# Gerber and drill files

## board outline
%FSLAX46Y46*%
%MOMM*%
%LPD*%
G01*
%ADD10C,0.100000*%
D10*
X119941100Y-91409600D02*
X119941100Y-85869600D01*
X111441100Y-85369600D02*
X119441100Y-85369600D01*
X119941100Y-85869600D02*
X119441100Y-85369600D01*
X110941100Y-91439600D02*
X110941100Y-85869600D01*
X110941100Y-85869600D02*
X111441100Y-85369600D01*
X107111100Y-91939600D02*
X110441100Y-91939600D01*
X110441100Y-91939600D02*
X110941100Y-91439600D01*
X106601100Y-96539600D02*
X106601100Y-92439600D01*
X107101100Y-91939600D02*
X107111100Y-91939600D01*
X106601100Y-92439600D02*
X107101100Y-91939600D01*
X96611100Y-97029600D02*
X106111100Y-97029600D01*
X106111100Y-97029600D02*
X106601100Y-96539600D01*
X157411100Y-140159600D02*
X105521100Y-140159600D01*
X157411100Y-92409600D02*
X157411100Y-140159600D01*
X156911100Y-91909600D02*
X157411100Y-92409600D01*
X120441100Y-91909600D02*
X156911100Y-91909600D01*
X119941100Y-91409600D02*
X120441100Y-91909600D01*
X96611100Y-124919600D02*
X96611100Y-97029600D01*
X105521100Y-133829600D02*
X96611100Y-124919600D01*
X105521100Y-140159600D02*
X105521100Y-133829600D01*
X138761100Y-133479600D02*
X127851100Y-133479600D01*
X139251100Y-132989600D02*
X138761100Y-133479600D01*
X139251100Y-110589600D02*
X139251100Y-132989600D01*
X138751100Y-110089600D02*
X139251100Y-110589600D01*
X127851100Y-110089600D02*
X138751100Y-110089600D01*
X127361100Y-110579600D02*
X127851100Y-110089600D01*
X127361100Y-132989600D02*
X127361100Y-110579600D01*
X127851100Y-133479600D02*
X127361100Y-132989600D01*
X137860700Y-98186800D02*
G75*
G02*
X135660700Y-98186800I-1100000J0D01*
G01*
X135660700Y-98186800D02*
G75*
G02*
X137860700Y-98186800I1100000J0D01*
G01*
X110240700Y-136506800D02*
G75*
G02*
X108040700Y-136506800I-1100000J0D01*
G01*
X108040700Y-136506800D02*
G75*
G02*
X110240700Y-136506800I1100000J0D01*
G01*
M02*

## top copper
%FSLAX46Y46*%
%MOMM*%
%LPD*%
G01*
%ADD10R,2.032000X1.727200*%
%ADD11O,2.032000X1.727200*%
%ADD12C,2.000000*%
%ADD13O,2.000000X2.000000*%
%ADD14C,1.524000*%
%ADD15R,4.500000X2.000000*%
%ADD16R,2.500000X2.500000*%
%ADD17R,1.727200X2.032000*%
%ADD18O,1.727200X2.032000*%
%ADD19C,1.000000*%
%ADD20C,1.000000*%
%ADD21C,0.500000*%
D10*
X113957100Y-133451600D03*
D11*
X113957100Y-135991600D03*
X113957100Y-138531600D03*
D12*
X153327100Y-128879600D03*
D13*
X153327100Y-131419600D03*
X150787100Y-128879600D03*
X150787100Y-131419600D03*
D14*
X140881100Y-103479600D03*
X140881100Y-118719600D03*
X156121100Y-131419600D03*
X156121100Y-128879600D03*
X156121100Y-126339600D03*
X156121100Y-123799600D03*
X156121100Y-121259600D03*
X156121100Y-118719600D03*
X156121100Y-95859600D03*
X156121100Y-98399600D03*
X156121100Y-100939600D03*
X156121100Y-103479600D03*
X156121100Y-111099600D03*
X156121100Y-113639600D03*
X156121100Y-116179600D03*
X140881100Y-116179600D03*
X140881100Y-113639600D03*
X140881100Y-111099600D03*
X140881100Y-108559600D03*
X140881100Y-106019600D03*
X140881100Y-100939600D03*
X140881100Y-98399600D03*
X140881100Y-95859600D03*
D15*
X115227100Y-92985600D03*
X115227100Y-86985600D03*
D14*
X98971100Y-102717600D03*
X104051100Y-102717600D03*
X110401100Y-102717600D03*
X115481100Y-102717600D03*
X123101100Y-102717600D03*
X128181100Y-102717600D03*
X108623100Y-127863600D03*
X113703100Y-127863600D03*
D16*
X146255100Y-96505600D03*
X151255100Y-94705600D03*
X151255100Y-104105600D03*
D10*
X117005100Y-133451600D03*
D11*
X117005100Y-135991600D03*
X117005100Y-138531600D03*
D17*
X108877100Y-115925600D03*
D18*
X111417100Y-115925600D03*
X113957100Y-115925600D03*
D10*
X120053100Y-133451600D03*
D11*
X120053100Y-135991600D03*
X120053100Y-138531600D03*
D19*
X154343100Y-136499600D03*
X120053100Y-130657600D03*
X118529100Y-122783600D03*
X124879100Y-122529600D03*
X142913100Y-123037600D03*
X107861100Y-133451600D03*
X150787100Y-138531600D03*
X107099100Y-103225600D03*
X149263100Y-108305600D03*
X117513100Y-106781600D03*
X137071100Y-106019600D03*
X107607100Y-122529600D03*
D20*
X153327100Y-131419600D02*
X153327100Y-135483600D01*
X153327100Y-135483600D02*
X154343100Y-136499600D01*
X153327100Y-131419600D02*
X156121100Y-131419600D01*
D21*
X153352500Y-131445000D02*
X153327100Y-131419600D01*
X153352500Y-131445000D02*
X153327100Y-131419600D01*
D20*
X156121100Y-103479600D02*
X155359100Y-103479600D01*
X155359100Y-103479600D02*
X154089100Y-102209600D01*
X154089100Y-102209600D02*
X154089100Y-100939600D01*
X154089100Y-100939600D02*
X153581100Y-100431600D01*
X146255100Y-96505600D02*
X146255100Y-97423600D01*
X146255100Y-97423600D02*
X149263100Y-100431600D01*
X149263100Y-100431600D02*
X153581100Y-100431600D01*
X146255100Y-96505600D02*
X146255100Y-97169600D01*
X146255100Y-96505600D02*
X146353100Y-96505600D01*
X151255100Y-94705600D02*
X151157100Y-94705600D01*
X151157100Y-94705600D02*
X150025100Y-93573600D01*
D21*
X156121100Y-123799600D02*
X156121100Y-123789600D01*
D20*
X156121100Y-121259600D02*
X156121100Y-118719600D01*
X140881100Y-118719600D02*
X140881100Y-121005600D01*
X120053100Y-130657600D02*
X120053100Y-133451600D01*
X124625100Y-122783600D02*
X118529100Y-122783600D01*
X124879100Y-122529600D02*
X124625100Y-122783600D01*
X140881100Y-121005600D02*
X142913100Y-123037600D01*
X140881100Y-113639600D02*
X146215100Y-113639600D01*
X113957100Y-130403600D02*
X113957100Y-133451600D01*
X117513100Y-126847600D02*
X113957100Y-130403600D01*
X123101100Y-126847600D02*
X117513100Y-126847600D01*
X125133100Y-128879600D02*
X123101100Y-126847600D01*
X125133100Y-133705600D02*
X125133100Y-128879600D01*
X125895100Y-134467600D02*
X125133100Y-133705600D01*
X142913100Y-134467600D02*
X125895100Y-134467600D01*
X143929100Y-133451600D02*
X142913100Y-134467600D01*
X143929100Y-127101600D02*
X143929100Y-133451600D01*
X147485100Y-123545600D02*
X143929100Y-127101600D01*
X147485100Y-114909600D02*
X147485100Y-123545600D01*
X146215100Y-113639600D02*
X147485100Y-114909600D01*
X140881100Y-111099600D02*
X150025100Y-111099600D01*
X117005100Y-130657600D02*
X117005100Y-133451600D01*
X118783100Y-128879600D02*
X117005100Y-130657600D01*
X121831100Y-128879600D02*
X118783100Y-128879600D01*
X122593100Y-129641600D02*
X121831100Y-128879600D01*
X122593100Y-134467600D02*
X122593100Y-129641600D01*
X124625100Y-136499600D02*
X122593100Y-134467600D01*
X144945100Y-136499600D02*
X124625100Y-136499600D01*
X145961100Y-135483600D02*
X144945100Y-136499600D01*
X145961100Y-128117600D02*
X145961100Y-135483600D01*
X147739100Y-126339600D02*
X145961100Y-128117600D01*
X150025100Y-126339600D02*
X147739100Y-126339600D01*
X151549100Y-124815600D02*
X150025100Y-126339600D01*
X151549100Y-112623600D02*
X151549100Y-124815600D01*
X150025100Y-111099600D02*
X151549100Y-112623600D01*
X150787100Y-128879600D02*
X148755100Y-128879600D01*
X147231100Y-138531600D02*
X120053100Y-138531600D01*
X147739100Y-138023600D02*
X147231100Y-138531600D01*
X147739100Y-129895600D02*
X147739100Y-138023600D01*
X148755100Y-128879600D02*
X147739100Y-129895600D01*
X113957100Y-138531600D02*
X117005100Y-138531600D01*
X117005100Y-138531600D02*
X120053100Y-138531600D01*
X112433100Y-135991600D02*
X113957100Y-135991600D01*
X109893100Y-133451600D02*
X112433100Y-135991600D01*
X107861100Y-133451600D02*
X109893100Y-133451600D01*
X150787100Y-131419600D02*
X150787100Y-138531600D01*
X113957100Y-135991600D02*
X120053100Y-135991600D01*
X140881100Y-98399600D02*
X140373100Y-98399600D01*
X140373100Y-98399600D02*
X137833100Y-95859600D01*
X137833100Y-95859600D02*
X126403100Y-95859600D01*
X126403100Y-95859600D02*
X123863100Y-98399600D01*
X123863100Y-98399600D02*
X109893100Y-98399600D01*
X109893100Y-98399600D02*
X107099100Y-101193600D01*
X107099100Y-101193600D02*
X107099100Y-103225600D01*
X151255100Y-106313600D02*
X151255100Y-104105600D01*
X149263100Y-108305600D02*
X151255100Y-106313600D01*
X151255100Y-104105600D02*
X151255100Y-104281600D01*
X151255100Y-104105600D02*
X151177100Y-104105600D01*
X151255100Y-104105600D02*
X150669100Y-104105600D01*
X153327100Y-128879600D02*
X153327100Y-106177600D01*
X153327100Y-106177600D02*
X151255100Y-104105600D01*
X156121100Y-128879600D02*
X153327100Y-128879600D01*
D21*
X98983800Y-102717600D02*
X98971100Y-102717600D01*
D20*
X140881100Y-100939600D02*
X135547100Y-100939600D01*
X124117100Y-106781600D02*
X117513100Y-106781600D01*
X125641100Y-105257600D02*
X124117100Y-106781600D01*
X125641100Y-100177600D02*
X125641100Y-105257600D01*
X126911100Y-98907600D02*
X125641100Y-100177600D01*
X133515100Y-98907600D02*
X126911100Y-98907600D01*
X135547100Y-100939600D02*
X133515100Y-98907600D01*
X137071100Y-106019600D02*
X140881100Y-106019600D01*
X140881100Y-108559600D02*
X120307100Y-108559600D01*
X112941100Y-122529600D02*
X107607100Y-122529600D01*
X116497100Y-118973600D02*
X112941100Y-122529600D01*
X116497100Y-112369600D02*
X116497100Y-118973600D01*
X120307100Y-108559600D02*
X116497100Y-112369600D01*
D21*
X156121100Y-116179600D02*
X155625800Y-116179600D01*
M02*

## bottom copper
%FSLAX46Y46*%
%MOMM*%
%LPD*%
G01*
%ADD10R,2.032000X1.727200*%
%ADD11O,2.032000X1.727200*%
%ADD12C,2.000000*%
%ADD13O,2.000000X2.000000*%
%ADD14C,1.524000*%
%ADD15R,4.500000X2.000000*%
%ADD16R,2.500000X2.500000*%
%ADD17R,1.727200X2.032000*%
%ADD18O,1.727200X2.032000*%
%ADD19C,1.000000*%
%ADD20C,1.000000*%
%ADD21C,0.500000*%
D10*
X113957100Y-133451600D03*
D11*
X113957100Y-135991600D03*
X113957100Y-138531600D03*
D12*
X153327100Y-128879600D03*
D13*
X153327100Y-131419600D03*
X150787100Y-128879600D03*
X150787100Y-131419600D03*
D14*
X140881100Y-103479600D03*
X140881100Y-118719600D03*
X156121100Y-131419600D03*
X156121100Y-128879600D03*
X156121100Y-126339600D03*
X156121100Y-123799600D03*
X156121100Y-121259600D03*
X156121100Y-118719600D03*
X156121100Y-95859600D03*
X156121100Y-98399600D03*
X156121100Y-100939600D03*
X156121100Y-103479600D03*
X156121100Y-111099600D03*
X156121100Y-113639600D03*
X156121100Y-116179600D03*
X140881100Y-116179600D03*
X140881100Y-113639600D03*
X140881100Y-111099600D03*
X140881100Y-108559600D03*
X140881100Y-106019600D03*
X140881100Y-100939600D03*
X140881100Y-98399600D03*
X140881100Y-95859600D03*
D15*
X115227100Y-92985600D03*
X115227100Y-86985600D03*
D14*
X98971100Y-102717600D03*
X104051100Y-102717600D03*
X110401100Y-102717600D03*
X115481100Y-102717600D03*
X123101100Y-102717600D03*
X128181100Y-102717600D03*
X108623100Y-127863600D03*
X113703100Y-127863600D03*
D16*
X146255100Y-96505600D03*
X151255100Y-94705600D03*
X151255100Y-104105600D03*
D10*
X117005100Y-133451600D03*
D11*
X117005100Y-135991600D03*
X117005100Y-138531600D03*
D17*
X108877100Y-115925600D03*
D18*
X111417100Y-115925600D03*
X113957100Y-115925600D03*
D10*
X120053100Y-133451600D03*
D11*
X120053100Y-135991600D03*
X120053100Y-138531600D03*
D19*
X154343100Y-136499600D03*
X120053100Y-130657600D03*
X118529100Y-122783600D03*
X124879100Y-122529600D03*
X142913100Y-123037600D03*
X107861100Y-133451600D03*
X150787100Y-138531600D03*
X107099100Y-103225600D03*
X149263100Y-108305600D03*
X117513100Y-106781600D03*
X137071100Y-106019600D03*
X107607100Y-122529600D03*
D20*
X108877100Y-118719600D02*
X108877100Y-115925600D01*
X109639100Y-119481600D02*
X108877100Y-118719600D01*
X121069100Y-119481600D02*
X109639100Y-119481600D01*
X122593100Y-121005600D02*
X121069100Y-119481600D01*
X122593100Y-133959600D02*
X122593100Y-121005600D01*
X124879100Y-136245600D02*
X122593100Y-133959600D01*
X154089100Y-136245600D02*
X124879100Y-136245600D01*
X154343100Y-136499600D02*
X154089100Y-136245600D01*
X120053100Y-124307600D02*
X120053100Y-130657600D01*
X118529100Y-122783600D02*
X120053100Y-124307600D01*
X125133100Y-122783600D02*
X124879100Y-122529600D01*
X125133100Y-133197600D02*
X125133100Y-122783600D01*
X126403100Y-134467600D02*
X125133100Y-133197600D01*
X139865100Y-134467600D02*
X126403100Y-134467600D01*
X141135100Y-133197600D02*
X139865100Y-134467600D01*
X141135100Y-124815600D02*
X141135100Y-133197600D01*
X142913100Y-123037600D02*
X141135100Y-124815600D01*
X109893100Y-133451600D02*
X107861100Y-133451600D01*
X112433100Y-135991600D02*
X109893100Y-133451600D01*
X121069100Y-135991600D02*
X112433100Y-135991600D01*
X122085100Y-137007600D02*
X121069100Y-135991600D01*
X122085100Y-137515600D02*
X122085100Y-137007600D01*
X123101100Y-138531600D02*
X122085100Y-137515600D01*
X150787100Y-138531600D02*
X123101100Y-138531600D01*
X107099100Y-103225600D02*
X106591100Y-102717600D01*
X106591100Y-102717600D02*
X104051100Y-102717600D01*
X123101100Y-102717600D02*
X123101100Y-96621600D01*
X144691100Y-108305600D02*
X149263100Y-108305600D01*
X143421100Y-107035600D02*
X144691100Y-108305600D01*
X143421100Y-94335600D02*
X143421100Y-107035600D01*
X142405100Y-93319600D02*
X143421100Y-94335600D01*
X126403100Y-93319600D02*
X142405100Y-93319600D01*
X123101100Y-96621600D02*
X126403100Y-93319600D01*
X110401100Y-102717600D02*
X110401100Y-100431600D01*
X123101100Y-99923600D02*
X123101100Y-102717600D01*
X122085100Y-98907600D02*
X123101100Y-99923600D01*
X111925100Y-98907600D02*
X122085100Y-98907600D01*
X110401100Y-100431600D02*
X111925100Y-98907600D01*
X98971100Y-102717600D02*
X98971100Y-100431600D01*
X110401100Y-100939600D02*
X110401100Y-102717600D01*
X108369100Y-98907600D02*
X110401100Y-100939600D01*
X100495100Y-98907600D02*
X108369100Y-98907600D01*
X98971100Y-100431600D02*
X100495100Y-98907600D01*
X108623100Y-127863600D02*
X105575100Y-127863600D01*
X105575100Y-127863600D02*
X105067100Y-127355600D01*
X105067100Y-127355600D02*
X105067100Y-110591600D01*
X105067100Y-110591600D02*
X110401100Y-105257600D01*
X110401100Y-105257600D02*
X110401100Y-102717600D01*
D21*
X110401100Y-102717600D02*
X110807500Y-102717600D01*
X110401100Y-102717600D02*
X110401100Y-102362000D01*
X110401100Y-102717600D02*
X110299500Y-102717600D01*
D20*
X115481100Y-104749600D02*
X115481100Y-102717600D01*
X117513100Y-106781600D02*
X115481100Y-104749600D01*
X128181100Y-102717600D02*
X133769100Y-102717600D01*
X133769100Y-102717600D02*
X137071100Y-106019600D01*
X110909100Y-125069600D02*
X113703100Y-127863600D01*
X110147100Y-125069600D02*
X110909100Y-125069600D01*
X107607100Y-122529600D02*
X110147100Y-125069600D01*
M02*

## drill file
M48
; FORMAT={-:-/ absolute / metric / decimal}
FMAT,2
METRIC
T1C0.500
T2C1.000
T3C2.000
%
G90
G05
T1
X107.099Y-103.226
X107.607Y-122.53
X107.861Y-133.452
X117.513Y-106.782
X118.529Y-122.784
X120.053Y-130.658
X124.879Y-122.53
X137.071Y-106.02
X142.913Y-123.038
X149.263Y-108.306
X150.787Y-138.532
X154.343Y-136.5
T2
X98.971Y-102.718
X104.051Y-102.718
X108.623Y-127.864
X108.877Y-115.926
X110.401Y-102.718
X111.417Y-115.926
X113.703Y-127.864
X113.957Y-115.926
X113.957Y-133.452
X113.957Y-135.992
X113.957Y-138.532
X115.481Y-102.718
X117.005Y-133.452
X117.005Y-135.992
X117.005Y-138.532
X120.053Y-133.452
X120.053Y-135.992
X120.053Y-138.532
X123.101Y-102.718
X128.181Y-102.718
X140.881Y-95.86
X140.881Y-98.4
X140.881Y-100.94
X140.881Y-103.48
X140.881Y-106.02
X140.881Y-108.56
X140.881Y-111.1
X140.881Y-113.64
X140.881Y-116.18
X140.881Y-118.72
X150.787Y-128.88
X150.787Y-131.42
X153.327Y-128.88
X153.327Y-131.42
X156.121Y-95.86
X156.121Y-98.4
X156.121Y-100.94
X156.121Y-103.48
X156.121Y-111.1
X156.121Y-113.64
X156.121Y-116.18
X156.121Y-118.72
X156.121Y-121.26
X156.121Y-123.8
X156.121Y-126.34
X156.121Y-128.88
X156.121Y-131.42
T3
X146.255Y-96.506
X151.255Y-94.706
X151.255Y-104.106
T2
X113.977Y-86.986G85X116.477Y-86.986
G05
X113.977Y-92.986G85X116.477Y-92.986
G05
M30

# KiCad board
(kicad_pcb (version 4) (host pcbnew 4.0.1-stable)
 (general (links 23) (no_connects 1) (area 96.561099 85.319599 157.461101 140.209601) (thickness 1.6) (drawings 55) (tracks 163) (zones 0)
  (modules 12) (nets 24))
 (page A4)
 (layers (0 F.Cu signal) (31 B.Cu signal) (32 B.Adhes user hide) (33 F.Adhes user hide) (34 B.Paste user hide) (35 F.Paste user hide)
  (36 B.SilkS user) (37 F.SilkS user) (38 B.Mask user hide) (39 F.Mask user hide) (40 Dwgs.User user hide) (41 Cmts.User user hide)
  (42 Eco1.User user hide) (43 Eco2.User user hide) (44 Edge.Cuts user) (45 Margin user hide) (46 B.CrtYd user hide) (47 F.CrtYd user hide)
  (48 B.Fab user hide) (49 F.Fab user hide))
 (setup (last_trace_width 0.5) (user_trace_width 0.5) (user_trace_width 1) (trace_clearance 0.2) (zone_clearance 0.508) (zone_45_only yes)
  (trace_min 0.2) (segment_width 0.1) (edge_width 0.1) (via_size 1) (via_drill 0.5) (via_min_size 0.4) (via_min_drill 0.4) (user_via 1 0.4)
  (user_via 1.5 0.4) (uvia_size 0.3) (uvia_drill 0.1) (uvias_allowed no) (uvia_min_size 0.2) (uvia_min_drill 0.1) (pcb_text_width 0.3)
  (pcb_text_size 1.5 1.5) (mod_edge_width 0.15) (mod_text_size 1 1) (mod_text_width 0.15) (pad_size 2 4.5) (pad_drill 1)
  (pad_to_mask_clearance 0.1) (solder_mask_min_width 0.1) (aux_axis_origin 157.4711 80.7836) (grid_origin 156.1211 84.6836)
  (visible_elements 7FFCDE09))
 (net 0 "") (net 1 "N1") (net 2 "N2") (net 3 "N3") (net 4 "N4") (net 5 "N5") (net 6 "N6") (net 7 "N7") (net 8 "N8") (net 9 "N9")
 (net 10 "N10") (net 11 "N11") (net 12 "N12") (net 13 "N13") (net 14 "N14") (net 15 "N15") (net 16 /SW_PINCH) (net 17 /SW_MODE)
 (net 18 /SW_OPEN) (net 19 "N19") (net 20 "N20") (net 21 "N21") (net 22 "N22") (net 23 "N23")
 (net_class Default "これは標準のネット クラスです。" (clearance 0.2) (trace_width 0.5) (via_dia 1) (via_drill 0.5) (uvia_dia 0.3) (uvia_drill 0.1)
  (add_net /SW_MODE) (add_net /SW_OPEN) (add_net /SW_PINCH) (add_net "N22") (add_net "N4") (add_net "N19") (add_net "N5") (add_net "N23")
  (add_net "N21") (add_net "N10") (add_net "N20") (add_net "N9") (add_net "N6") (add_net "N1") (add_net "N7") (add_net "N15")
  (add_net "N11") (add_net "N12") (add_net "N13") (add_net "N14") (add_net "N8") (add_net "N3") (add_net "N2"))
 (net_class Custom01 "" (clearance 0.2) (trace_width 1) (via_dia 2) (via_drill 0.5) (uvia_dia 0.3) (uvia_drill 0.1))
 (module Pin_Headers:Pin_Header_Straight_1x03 (layer F.Cu) (at 113.9571 133.4516)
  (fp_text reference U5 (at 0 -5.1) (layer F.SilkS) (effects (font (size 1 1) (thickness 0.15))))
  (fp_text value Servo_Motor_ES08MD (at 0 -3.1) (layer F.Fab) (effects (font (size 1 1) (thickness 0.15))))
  (pad 1 thru_hole rect (at 0 0) (size 2.032 1.7272) (drill 1) (layers *.Cu *.Mask F.SilkS) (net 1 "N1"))
  (pad 2 thru_hole oval (at 0 2.54) (size 2.032 1.7272) (drill 1) (layers *.Cu *.Mask F.SilkS) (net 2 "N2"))
  (pad 3 thru_hole oval (at 0 5.08) (size 2.032 1.7272) (drill 1) (layers *.Cu *.Mask F.SilkS) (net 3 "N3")))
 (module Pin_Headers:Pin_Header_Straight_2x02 (layer F.Cu) (at 153.3271 128.8796 270)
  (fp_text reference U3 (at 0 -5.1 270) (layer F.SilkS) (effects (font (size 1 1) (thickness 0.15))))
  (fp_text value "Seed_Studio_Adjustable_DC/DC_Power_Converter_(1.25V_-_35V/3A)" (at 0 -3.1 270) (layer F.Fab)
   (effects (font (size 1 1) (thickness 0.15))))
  (pad 2 thru_hole circle (at 0 0 270) (size 2 2) (drill 1) (layers *.Cu *.Mask F.SilkS) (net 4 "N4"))
  (pad 1 thru_hole oval (at 2.54 0 270) (size 2 2) (drill 1) (layers *.Cu *.Mask F.SilkS) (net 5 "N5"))
  (pad 3 thru_hole oval (at 0 2.54 270) (size 2 2) (drill 1) (layers *.Cu *.Mask F.SilkS) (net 3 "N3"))
  (pad 4 thru_hole oval (at 2.54 2.54 270) (size 2 2) (drill 1) (layers *.Cu *.Mask F.SilkS) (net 2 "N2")))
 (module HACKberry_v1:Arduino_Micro (layer F.Cu) (at 148.5011 116.1796 180)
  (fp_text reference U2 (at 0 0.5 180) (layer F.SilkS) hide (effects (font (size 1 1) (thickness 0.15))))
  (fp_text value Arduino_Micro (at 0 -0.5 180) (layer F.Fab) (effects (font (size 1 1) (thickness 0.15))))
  (pad 9 thru_hole circle (at 7.62 12.7 180) (size 1.524 1.524) (drill 1) (layers *.Cu *.Mask F.SilkS))
  (pad 3 thru_hole circle (at 7.62 -2.54 180) (size 1.524 1.524) (drill 1) (layers *.Cu *.Mask F.SilkS) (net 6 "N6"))
  (pad VIN thru_hole circle (at -7.62 -15.24 180) (size 1.524 1.524) (drill 1) (layers *.Cu *.Mask F.SilkS) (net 5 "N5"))
  (pad GND thru_hole circle (at -7.62 -12.7 180) (size 1.524 1.524) (drill 1) (layers *.Cu *.Mask F.SilkS) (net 4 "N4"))
  (pad eRST thru_hole circle (at -7.62 -10.16 180) (size 1.524 1.524) (drill 1) (layers *.Cu *.Mask F.SilkS))
  (pad 5V thru_hole circle (at -7.62 -7.62 180) (size 1.524 1.524) (drill 1) (layers *.Cu *.Mask F.SilkS) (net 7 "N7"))
  (pad NC thru_hole circle (at -7.62 -5.08 180) (size 1.524 1.524) (drill 1) (layers *.Cu *.Mask F.SilkS) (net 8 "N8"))
  (pad NC thru_hole circle (at -7.62 -2.54 180) (size 1.524 1.524) (drill 1) (layers *.Cu *.Mask F.SilkS) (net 8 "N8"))
  (pad 13 thru_hole circle (at -7.62 20.32 180) (size 1.524 1.524) (drill 1) (layers *.Cu *.Mask F.SilkS) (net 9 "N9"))
  (pad 3.3V thru_hole circle (at -7.62 17.78 180) (size 1.524 1.524) (drill 1) (layers *.Cu *.Mask F.SilkS))
  (pad AREF thru_hole circle (at -7.62 15.24 180) (size 1.524 1.524) (drill 1) (layers *.Cu *.Mask F.SilkS))
  (pad A0 thru_hole circle (at -7.62 12.7 180) (size 1.524 1.524) (drill 1) (layers *.Cu *.Mask F.SilkS) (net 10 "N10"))
  (pad A3 thru_hole circle (at -7.62 5.08 180) (size 1.524 1.524) (drill 1) (layers *.Cu *.Mask F.SilkS) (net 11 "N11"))
  (pad A4 thru_hole circle (at -7.62 2.54 180) (size 1.524 1.524) (drill 1) (layers *.Cu *.Mask F.SilkS) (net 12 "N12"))
  (pad A5 thru_hole circle (at -7.62 0 180) (size 1.524 1.524) (drill 1) (layers *.Cu *.Mask F.SilkS) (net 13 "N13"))
  (pad A6 thru_hole circle (at 7.62 0 180) (size 1.524 1.524) (drill 1) (layers *.Cu *.Mask F.SilkS) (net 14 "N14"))
  (pad 5 thru_hole circle (at 7.62 2.54 180) (size 1.524 1.524) (drill 1) (layers *.Cu *.Mask F.SilkS) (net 1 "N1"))
  (pad 6 thru_hole circle (at 7.62 5.08 180) (size 1.524 1.524) (drill 1) (layers *.Cu *.Mask F.SilkS) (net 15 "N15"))
  (pad 7 thru_hole circle (at 7.62 7.62 180) (size 1.524 1.524) (drill 1) (layers *.Cu *.Mask F.SilkS) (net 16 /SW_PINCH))
  (pad 8 thru_hole circle (at 7.62 10.16 180) (size 1.524 1.524) (drill 1) (layers *.Cu *.Mask F.SilkS) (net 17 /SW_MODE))
  (pad 10 thru_hole circle (at 7.62 15.24 180) (size 1.524 1.524) (drill 1) (layers *.Cu *.Mask F.SilkS) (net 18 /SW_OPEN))
  (pad 11 thru_hole circle (at 7.62 17.78 180) (size 1.524 1.524) (drill 1) (layers *.Cu *.Mask F.SilkS) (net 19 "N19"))
  (pad 12 thru_hole circle (at 7.62 20.32 180) (size 1.524 1.524) (drill 1) (layers *.Cu *.Mask F.SilkS) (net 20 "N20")))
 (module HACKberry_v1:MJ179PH (layer F.Cu) (at 115.2271 100.6856 90)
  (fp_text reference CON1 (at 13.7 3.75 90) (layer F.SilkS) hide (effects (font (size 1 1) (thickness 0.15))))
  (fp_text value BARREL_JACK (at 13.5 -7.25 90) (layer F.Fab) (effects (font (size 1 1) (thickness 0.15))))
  (pad "" thru_hole rect (at 7.7 0 90) (size 2 4.5) (drill oval 1 3.5) (layers *.Cu *.Mask F.SilkS))
  (pad "" thru_hole rect (at 13.7 0 90) (size 2 4.5) (drill oval 1 3.5) (layers *.Cu *.Mask F.SilkS)))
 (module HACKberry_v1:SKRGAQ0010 (layer F.Cu) (at 101.5111 102.7176 90)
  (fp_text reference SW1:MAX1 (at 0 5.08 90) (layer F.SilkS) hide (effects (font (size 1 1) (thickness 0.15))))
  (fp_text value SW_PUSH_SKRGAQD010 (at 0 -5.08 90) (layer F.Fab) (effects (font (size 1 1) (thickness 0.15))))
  (pad 1 thru_hole circle (at 0 -2.54 90) (size 1.524 1.524) (drill 1) (layers *.Cu *.Mask F.SilkS) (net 4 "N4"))
  (pad 2 thru_hole circle (at 0 2.54 90) (size 1.524 1.524) (drill 1) (layers *.Cu *.Mask F.SilkS) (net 19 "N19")))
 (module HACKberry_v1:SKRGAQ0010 (layer F.Cu) (at 112.9411 102.7176 90)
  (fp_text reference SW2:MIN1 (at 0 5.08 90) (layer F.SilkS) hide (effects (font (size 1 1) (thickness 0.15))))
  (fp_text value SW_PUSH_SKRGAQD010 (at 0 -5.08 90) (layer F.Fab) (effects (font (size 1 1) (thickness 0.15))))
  (pad 1 thru_hole circle (at 0 -2.54 90) (size 1.524 1.524) (drill 1) (layers *.Cu *.Mask F.SilkS) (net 4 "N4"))
  (pad 2 thru_hole circle (at 0 2.54 90) (size 1.524 1.524) (drill 1) (layers *.Cu *.Mask F.SilkS) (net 18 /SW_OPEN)))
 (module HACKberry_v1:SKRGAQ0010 (layer F.Cu) (at 125.6411 102.7176 90)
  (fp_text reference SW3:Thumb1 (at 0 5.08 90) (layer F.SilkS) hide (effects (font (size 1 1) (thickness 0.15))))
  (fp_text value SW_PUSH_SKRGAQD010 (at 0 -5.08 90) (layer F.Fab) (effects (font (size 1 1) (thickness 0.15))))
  (pad 1 thru_hole circle (at 0 -2.54 90) (size 1.524 1.524) (drill 1) (layers *.Cu *.Mask F.SilkS) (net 4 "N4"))
  (pad 2 thru_hole circle (at 0 2.54 90) (size 1.524 1.524) (drill 1) (layers *.Cu *.Mask F.SilkS) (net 17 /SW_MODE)))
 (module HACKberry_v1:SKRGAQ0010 (layer F.Cu) (at 111.1631 127.8636 90)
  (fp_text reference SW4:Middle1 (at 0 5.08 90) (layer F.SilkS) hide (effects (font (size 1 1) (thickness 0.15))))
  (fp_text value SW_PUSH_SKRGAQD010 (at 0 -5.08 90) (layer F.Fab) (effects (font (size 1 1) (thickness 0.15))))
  (pad 1 thru_hole circle (at 0 -2.54 90) (size 1.524 1.524) (drill 1) (layers *.Cu *.Mask F.SilkS) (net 4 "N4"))
  (pad 2 thru_hole circle (at 0 2.54 90) (size 1.524 1.524) (drill 1) (layers *.Cu *.Mask F.SilkS) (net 16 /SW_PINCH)))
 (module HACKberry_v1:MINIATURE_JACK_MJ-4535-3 (layer F.Cu) (at 148.7551 95.6056 90)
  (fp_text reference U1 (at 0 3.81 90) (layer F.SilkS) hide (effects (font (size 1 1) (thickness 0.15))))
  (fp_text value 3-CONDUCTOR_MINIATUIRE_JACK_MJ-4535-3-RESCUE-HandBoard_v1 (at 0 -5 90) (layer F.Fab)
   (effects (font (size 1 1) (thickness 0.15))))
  (pad 4 thru_hole rect (at -0.9 -2.5 90) (size 2.5 2.5) (drill oval 2) (layers *.Cu *.Mask F.SilkS) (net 10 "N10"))
  (pad 2 thru_hole rect (at 0.9 2.5 90) (size 2.5 2.5) (drill oval 2) (layers *.Cu *.Mask F.SilkS) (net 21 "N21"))
  (pad 1 thru_hole rect (at -8.5 2.5 90) (size 2.5 2.5) (drill oval 2) (layers *.Cu *.Mask F.SilkS) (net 4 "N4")))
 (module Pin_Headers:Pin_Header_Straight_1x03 (layer F.Cu) (at 117.0051 133.4516)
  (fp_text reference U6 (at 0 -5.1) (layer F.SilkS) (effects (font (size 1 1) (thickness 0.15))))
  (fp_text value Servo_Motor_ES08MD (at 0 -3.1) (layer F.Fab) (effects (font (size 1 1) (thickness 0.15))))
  (pad 1 thru_hole rect (at 0 0) (size 2.032 1.7272) (drill 1) (layers *.Cu *.Mask F.SilkS) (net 15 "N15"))
  (pad 2 thru_hole oval (at 0 2.54) (size 2.032 1.7272) (drill 1) (layers *.Cu *.Mask F.SilkS) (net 2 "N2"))
  (pad 3 thru_hole oval (at 0 5.08) (size 2.032 1.7272) (drill 1) (layers *.Cu *.Mask F.SilkS) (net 3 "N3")))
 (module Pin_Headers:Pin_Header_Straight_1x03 (layer F.Cu) (at 108.8771 115.9256 90)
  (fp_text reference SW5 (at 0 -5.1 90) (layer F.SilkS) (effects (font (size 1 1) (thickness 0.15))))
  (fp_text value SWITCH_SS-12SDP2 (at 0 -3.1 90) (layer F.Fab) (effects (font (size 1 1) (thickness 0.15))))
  (pad 1 thru_hole rect (at 0 0 90) (size 2.032 1.7272) (drill 1) (layers *.Cu *.Mask F.SilkS) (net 5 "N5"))
  (pad 2 thru_hole oval (at 0 2.54 90) (size 2.032 1.7272) (drill 1) (layers *.Cu *.Mask F.SilkS) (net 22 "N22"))
  (pad 3 thru_hole oval (at 0 5.08 90) (size 2.032 1.7272) (drill 1) (layers *.Cu *.Mask F.SilkS) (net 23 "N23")))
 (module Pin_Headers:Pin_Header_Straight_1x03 (layer F.Cu) (at 120.0531 133.4516)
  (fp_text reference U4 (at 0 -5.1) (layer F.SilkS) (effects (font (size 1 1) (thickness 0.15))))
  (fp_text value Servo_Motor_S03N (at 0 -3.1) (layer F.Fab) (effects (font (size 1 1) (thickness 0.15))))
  (pad 1 thru_hole rect (at 0 0) (size 2.032 1.7272) (drill 1) (layers *.Cu *.Mask F.SilkS) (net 6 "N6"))
  (pad 2 thru_hole oval (at 0 2.54) (size 2.032 1.7272) (drill 1) (layers *.Cu *.Mask F.SilkS) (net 2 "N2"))
  (pad 3 thru_hole oval (at 0 5.08) (size 2.032 1.7272) (drill 1) (layers *.Cu *.Mask F.SilkS) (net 3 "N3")))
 (gr_line (start 119.9411 91.4096) (end 119.9411 85.8696) (angle 90) (layer Edge.Cuts) (width 0.1))
 (gr_line (start 111.4411 85.3696) (end 119.4411 85.3696) (angle 90) (layer Edge.Cuts) (width 0.1))
 (gr_line (start 119.9411 85.8696) (end 119.4411 85.3696) (angle 90) (layer Edge.Cuts) (width 0.1))
 (gr_line (start 110.9411 91.4396) (end 110.9411 85.8696) (angle 90) (layer Edge.Cuts) (width 0.1))
 (gr_line (start 110.9411 85.8696) (end 111.4411 85.3696) (angle 90) (layer Edge.Cuts) (width 0.1))
 (gr_line (start 107.1111 91.9396) (end 110.4411 91.9396) (angle 90) (layer Edge.Cuts) (width 0.1))
 (gr_line (start 110.4411 91.9396) (end 110.9411 91.4396) (angle 90) (layer Edge.Cuts) (width 0.1))
 (gr_line (start 106.6011 96.5396) (end 106.6011 92.4396) (angle 90) (layer Edge.Cuts) (width 0.1))
 (gr_line (start 107.1011 91.9396) (end 107.1111 91.9396) (angle 90) (layer Edge.Cuts) (width 0.1))
 (gr_line (start 106.6011 92.4396) (end 107.1011 91.9396) (angle 90) (layer Edge.Cuts) (width 0.1))
 (gr_line (start 96.6111 97.0296) (end 106.1111 97.0296) (angle 90) (layer Edge.Cuts) (width 0.1))
 (gr_line (start 106.1111 97.0296) (end 106.6011 96.5396) (angle 90) (layer Edge.Cuts) (width 0.1))
 (gr_line (start 157.4111 140.1596) (end 105.5211 140.1596) (angle 90) (layer Edge.Cuts) (width 0.1))
 (gr_line (start 157.4111 92.4096) (end 157.4111 140.1596) (angle 90) (layer Edge.Cuts) (width 0.1))
 (gr_line (start 156.9111 91.9096) (end 157.4111 92.4096) (angle 90) (layer Edge.Cuts) (width 0.1))
 (gr_line (start 120.4411 91.9096) (end 156.9111 91.9096) (angle 90) (layer Edge.Cuts) (width 0.1))
 (gr_line (start 119.9411 91.4096) (end 120.4411 91.9096) (angle 90) (layer Edge.Cuts) (width 0.1))
 (gr_line (start 96.6111 124.9196) (end 96.6111 97.0296) (angle 90) (layer Edge.Cuts) (width 0.1))
 (gr_line (start 105.5211 133.8296) (end 96.6111 124.9196) (angle 90) (layer Edge.Cuts) (width 0.1))
 (gr_line (start 105.5211 140.1596) (end 105.5211 133.8296) (angle 90) (layer Edge.Cuts) (width 0.1))
 (gr_line (start 138.7611 133.4796) (end 127.8511 133.4796) (angle 90) (layer Edge.Cuts) (width 0.1))
 (gr_line (start 139.2511 132.9896) (end 138.7611 133.4796) (angle 90) (layer Edge.Cuts) (width 0.1))
 (gr_line (start 139.2511 110.5896) (end 139.2511 132.9896) (angle 90) (layer Edge.Cuts) (width 0.1))
 (gr_line (start 138.7511 110.0896) (end 139.2511 110.5896) (angle 90) (layer Edge.Cuts) (width 0.1))
 (gr_line (start 127.8511 110.0896) (end 138.7511 110.0896) (angle 90) (layer Edge.Cuts) (width 0.1))
 (gr_line (start 127.3611 110.5796) (end 127.8511 110.0896) (angle 90) (layer Edge.Cuts) (width 0.1))
 (gr_line (start 127.3611 132.9896) (end 127.3611 110.5796) (angle 90) (layer Edge.Cuts) (width 0.1))
 (gr_line (start 127.8511 133.4796) (end 127.3611 132.9896) (angle 90) (layer Edge.Cuts) (width 0.1))
 (gr_circle (center 136.7607 98.1868) (end 137.8607 98.1868) (layer Edge.Cuts) (width 0.1))
 (gr_circle (center 109.1407 136.5068) (end 110.2407 136.5068) (layer Edge.Cuts) (width 0.1))
 (segment (start 153.3271 131.4196) (end 153.3271 135.4836) (width 1) (layer F.Cu) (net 5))
 (segment (start 108.8771 118.7196) (end 108.8771 115.9256) (width 1) (layer B.Cu) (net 5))
 (segment (start 109.6391 119.4816) (end 108.8771 118.7196) (width 1) (layer B.Cu) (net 5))
 (segment (start 121.0691 119.4816) (end 109.6391 119.4816) (width 1) (layer B.Cu) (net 5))
 (segment (start 122.5931 121.0056) (end 121.0691 119.4816) (width 1) (layer B.Cu) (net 5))
 (segment (start 122.5931 133.9596) (end 122.5931 121.0056) (width 1) (layer B.Cu) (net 5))
 (segment (start 124.8791 136.2456) (end 122.5931 133.9596) (width 1) (layer B.Cu) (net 5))
 (segment (start 154.0891 136.2456) (end 124.8791 136.2456) (width 1) (layer B.Cu) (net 5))
 (segment (start 154.3431 136.4996) (end 154.0891 136.2456) (width 1) (layer B.Cu) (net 5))
 (via (at 154.3431 136.4996) (size 1) (drill 0.5) (layers F.Cu B.Cu) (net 5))
 (segment (start 153.3271 135.4836) (end 154.3431 136.4996) (width 1) (layer F.Cu) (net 5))
 (segment (start 153.3271 131.4196) (end 156.1211 131.4196) (width 1) (layer F.Cu) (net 5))
 (segment (start 153.3525 131.445) (end 153.3271 131.4196) (width 0.5) (layer F.Cu) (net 5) (status 30))
 (segment (start 153.3525 131.445) (end 153.3271 131.4196) (width 0.5) (layer F.Cu) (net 5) (status 30))
 (segment (start 156.1211 103.4796) (end 155.3591 103.4796) (width 1) (layer F.Cu) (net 10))
 (segment (start 155.3591 103.4796) (end 154.0891 102.2096) (width 1) (layer F.Cu) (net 10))
 (segment (start 154.0891 102.2096) (end 154.0891 100.9396) (width 1) (layer F.Cu) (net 10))
 (segment (start 154.0891 100.9396) (end 153.5811 100.4316) (width 1) (layer F.Cu) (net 10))
 (segment (start 146.2551 96.5056) (end 146.2551 97.4236) (width 1) (layer F.Cu) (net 10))
 (segment (start 146.2551 97.4236) (end 149.2631 100.4316) (width 1) (layer F.Cu) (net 10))
 (segment (start 149.2631 100.4316) (end 153.5811 100.4316) (width 1) (layer F.Cu) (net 10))
 (segment (start 146.2551 96.5056) (end 146.2551 97.1696) (width 1) (layer F.Cu) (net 10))
 (segment (start 146.2551 96.5056) (end 146.3531 96.5056) (width 1) (layer F.Cu) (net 10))
 (segment (start 151.2551 94.7056) (end 151.1571 94.7056) (width 1) (layer F.Cu) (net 21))
 (segment (start 151.1571 94.7056) (end 150.0251 93.5736) (width 1) (layer F.Cu) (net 21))
 (segment (start 156.1211 123.7996) (end 156.1211 123.7896) (width 0.5) (layer F.Cu) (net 7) (status 30))
 (segment (start 156.1211 121.2596) (end 156.1211 118.7196) (width 1) (layer F.Cu) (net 8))
 (segment (start 140.8811 118.7196) (end 140.8811 121.0056) (width 1) (layer F.Cu) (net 6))
 (segment (start 120.0531 130.6576) (end 120.0531 133.4516) (width 1) (layer F.Cu) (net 6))
 (via (at 120.0531 130.6576) (size 1) (drill 0.5) (layers F.Cu B.Cu) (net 6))
 (segment (start 120.0531 124.3076) (end 120.0531 130.6576) (width 1) (layer B.Cu) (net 6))
 (segment (start 118.5291 122.7836) (end 120.0531 124.3076) (width 1) (layer B.Cu) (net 6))
 (via (at 118.5291 122.7836) (size 1) (drill 0.5) (layers F.Cu B.Cu) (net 6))
 (segment (start 124.6251 122.7836) (end 118.5291 122.7836) (width 1) (layer F.Cu) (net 6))
 (segment (start 124.8791 122.5296) (end 124.6251 122.7836) (width 1) (layer F.Cu) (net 6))
 (via (at 124.8791 122.5296) (size 1) (drill 0.5) (layers F.Cu B.Cu) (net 6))
 (segment (start 125.1331 122.7836) (end 124.8791 122.5296) (width 1) (layer B.Cu) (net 6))
 (segment (start 125.1331 133.1976) (end 125.1331 122.7836) (width 1) (layer B.Cu) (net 6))
 (segment (start 126.4031 134.4676) (end 125.1331 133.1976) (width 1) (layer B.Cu) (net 6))
 (segment (start 139.8651 134.4676) (end 126.4031 134.4676) (width 1) (layer B.Cu) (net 6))
 (segment (start 141.1351 133.1976) (end 139.8651 134.4676) (width 1) (layer B.Cu) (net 6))
 (segment (start 141.1351 124.8156) (end 141.1351 133.1976) (width 1) (layer B.Cu) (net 6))
 (segment (start 142.9131 123.0376) (end 141.1351 124.8156) (width 1) (layer B.Cu) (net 6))
 (via (at 142.9131 123.0376) (size 1) (drill 0.5) (layers F.Cu B.Cu) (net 6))
 (segment (start 140.8811 121.0056) (end 142.9131 123.0376) (width 1) (layer F.Cu) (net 6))
 (segment (start 140.8811 113.6396) (end 146.2151 113.6396) (width 1) (layer F.Cu) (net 1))
 (segment (start 113.9571 130.4036) (end 113.9571 133.4516) (width 1) (layer F.Cu) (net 1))
 (segment (start 117.5131 126.8476) (end 113.9571 130.4036) (width 1) (layer F.Cu) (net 1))
 (segment (start 123.1011 126.8476) (end 117.5131 126.8476) (width 1) (layer F.Cu) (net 1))
 (segment (start 125.1331 128.8796) (end 123.1011 126.8476) (width 1) (layer F.Cu) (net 1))
 (segment (start 125.1331 133.7056) (end 125.1331 128.8796) (width 1) (layer F.Cu) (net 1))
 (segment (start 125.8951 134.4676) (end 125.1331 133.7056) (width 1) (layer F.Cu) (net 1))
 (segment (start 142.9131 134.4676) (end 125.8951 134.4676) (width 1) (layer F.Cu) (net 1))
 (segment (start 143.9291 133.4516) (end 142.9131 134.4676) (width 1) (layer F.Cu) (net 1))
 (segment (start 143.9291 127.1016) (end 143.9291 133.4516) (width 1) (layer F.Cu) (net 1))
 (segment (start 147.4851 123.5456) (end 143.9291 127.1016) (width 1) (layer F.Cu) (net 1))
 (segment (start 147.4851 114.9096) (end 147.4851 123.5456) (width 1) (layer F.Cu) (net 1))
 (segment (start 146.2151 113.6396) (end 147.4851 114.9096) (width 1) (layer F.Cu) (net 1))
 (segment (start 140.8811 111.0996) (end 150.0251 111.0996) (width 1) (layer F.Cu) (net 15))
 (segment (start 117.0051 130.6576) (end 117.0051 133.4516) (width 1) (layer F.Cu) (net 15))
 (segment (start 118.7831 128.8796) (end 117.0051 130.6576) (width 1) (layer F.Cu) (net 15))
 (segment (start 121.8311 128.8796) (end 118.7831 128.8796) (width 1) (layer F.Cu) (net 15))
 (segment (start 122.5931 129.6416) (end 121.8311 128.8796) (width 1) (layer F.Cu) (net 15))
 (segment (start 122.5931 134.4676) (end 122.5931 129.6416) (width 1) (layer F.Cu) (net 15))
 (segment (start 124.6251 136.4996) (end 122.5931 134.4676) (width 1) (layer F.Cu) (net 15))
 (segment (start 144.9451 136.4996) (end 124.6251 136.4996) (width 1) (layer F.Cu) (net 15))
 (segment (start 145.9611 135.4836) (end 144.9451 136.4996) (width 1) (layer F.Cu) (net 15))
 (segment (start 145.9611 128.1176) (end 145.9611 135.4836) (width 1) (layer F.Cu) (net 15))
 (segment (start 147.7391 126.3396) (end 145.9611 128.1176) (width 1) (layer F.Cu) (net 15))
 (segment (start 150.0251 126.3396) (end 147.7391 126.3396) (width 1) (layer F.Cu) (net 15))
 (segment (start 151.5491 124.8156) (end 150.0251 126.3396) (width 1) (layer F.Cu) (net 15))
 (segment (start 151.5491 112.6236) (end 151.5491 124.8156) (width 1) (layer F.Cu) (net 15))
 (segment (start 150.0251 111.0996) (end 151.5491 112.6236) (width 1) (layer F.Cu) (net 15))
 (segment (start 150.7871 128.8796) (end 148.7551 128.8796) (width 1) (layer F.Cu) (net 3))
 (segment (start 147.2311 138.5316) (end 120.0531 138.5316) (width 1) (layer F.Cu) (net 3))
 (segment (start 147.7391 138.0236) (end 147.2311 138.5316) (width 1) (layer F.Cu) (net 3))
 (segment (start 147.7391 129.8956) (end 147.7391 138.0236) (width 1) (layer F.Cu) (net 3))
 (segment (start 148.7551 128.8796) (end 147.7391 129.8956) (width 1) (layer F.Cu) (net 3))
 (segment (start 113.9571 138.5316) (end 117.0051 138.5316) (width 1) (layer F.Cu) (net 3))
 (segment (start 117.0051 138.5316) (end 120.0531 138.5316) (width 1) (layer F.Cu) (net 3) (status 20))
 (segment (start 112.4331 135.9916) (end 113.9571 135.9916) (width 1) (layer F.Cu) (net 2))
 (segment (start 109.8931 133.4516) (end 112.4331 135.9916) (width 1) (layer F.Cu) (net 2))
 (segment (start 107.8611 133.4516) (end 109.8931 133.4516) (width 1) (layer F.Cu) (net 2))
 (via (at 107.8611 133.4516) (size 1) (drill 0.5) (layers F.Cu B.Cu) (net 2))
 (segment (start 109.8931 133.4516) (end 107.8611 133.4516) (width 1) (layer B.Cu) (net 2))
 (segment (start 112.4331 135.9916) (end 109.8931 133.4516) (width 1) (layer B.Cu) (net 2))
 (segment (start 121.0691 135.9916) (end 112.4331 135.9916) (width 1) (layer B.Cu) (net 2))
 (segment (start 122.0851 137.0076) (end 121.0691 135.9916) (width 1) (layer B.Cu) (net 2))
 (segment (start 122.0851 137.5156) (end 122.0851 137.0076) (width 1) (layer B.Cu) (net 2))
 (segment (start 123.1011 138.5316) (end 122.0851 137.5156) (width 1) (layer B.Cu) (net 2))
 (segment (start 150.7871 138.5316) (end 123.1011 138.5316) (width 1) (layer B.Cu) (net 2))
 (via (at 150.7871 138.5316) (size 1) (drill 0.5) (layers F.Cu B.Cu) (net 2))
 (segment (start 150.7871 131.4196) (end 150.7871 138.5316) (width 1) (layer F.Cu) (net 2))
 (segment (start 113.9571 135.9916) (end 120.0531 135.9916) (width 1) (layer F.Cu) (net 2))
 (segment (start 140.8811 98.3996) (end 140.3731 98.3996) (width 1) (layer F.Cu) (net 19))
 (segment (start 140.3731 98.3996) (end 137.8331 95.8596) (width 1) (layer F.Cu) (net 19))
 (segment (start 137.8331 95.8596) (end 126.4031 95.8596) (width 1) (layer F.Cu) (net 19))
 (segment (start 126.4031 95.8596) (end 123.8631 98.3996) (width 1) (layer F.Cu) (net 19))
 (segment (start 123.8631 98.3996) (end 109.8931 98.3996) (width 1) (layer F.Cu) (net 19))
 (segment (start 109.8931 98.3996) (end 107.0991 101.1936) (width 1) (layer F.Cu) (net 19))
 (segment (start 107.0991 101.1936) (end 107.0991 103.2256) (width 1) (layer F.Cu) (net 19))
 (via (at 107.0991 103.2256) (size 1) (drill 0.5) (layers F.Cu B.Cu) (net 19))
 (segment (start 107.0991 103.2256) (end 106.5911 102.7176) (width 1) (layer B.Cu) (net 19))
 (segment (start 106.5911 102.7176) (end 104.0511 102.7176) (width 1) (layer B.Cu) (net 19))
 (segment (start 123.1011 102.7176) (end 123.1011 96.6216) (width 1) (layer B.Cu) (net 4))
 (segment (start 151.2551 106.3136) (end 151.2551 104.1056) (width 1) (layer F.Cu) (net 4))
 (segment (start 149.2631 108.3056) (end 151.2551 106.3136) (width 1) (layer F.Cu) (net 4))
 (via (at 149.2631 108.3056) (size 1) (drill 0.5) (layers F.Cu B.Cu) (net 4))
 (segment (start 144.6911 108.3056) (end 149.2631 108.3056) (width 1) (layer B.Cu) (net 4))
 (segment (start 143.4211 107.0356) (end 144.6911 108.3056) (width 1) (layer B.Cu) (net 4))
 (segment (start 143.4211 94.3356) (end 143.4211 107.0356) (width 1) (layer B.Cu) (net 4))
 (segment (start 142.4051 93.3196) (end 143.4211 94.3356) (width 1) (layer B.Cu) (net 4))
 (segment (start 126.4031 93.3196) (end 142.4051 93.3196) (width 1) (layer B.Cu) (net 4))
 (segment (start 123.1011 96.6216) (end 126.4031 93.3196) (width 1) (layer B.Cu) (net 4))
 (segment (start 110.4011 102.7176) (end 110.4011 100.4316) (width 1) (layer B.Cu) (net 4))
 (segment (start 123.1011 99.9236) (end 123.1011 102.7176) (width 1) (layer B.Cu) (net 4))
 (segment (start 122.0851 98.9076) (end 123.1011 99.9236) (width 1) (layer B.Cu) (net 4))
 (segment (start 111.9251 98.9076) (end 122.0851 98.9076) (width 1) (layer B.Cu) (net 4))
 (segment (start 110.4011 100.4316) (end 111.9251 98.9076) (width 1) (layer B.Cu) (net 4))
 (segment (start 98.9711 102.7176) (end 98.9711 100.4316) (width 1) (layer B.Cu) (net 4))
 (segment (start 110.4011 100.9396) (end 110.4011 102.7176) (width 1) (layer B.Cu) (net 4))
 (segment (start 108.3691 98.9076) (end 110.4011 100.9396) (width 1) (layer B.Cu) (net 4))
 (segment (start 100.4951 98.9076) (end 108.3691 98.9076) (width 1) (layer B.Cu) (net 4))
 (segment (start 98.9711 100.4316) (end 100.4951 98.9076) (width 1) (layer B.Cu) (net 4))
 (segment (start 151.2551 104.1056) (end 151.2551 104.2816) (width 1) (layer F.Cu) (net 4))
 (segment (start 151.2551 104.1056) (end 151.1771 104.1056) (width 1) (layer F.Cu) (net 4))
 (segment (start 108.6231 127.8636) (end 105.5751 127.8636) (width 1) (layer B.Cu) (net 4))
 (segment (start 105.5751 127.8636) (end 105.0671 127.3556) (width 1) (layer B.Cu) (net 4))
 (segment (start 105.0671 127.3556) (end 105.0671 110.5916) (width 1) (layer B.Cu) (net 4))
 (segment (start 105.0671 110.5916) (end 110.4011 105.2576) (width 1) (layer B.Cu) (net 4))
 (segment (start 110.4011 105.2576) (end 110.4011 102.7176) (width 1) (layer B.Cu) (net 4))
 (segment (start 151.2551 104.1056) (end 150.6691 104.1056) (width 1) (layer F.Cu) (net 4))
 (segment (start 153.3271 128.8796) (end 153.3271 106.1776) (width 1) (layer F.Cu) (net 4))
 (segment (start 153.3271 106.1776) (end 151.2551 104.1056) (width 1) (layer F.Cu) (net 4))
 (segment (start 156.1211 128.8796) (end 153.3271 128.8796) (width 1) (layer F.Cu) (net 4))
 (segment (start 110.4011 102.7176) (end 110.8075 102.7176) (width 0.5) (layer B.Cu) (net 4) (status 30))
 (segment (start 110.4011 102.7176) (end 110.4011 102.362) (width 0.5) (layer B.Cu) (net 4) (status 30))
 (segment (start 110.4011 102.7176) (end 110.2995 102.7176) (width 0.5) (layer B.Cu) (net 4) (status 30))
 (segment (start 98.9838 102.7176) (end 98.9711 102.7176) (width 0.5) (layer F.Cu) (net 4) (status 30))
 (segment (start 140.8811 100.9396) (end 135.5471 100.9396) (width 1) (layer F.Cu) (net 18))
 (segment (start 115.4811 104.7496) (end 115.4811 102.7176) (width 1) (layer B.Cu) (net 18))
 (segment (start 117.5131 106.7816) (end 115.4811 104.7496) (width 1) (layer B.Cu) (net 18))
 (via (at 117.5131 106.7816) (size 1) (drill 0.5) (layers F.Cu B.Cu) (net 18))
 (segment (start 124.1171 106.7816) (end 117.5131 106.7816) (width 1) (layer F.Cu) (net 18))
 (segment (start 125.6411 105.2576) (end 124.1171 106.7816) (width 1) (layer F.Cu) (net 18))
 (segment (start 125.6411 100.1776) (end 125.6411 105.2576) (width 1) (layer F.Cu) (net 18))
 (segment (start 126.9111 98.9076) (end 125.6411 100.1776) (width 1) (layer F.Cu) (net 18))
 (segment (start 133.5151 98.9076) (end 126.9111 98.9076) (width 1) (layer F.Cu) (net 18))
 (segment (start 135.5471 100.9396) (end 133.5151 98.9076) (width 1) (layer F.Cu) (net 18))
 (segment (start 128.1811 102.7176) (end 133.7691 102.7176) (width 1) (layer B.Cu) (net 17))
 (segment (start 137.0711 106.0196) (end 140.8811 106.0196) (width 1) (layer F.Cu) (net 17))
 (via (at 137.0711 106.0196) (size 1) (drill 0.5) (layers F.Cu B.Cu) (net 17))
 (segment (start 133.7691 102.7176) (end 137.0711 106.0196) (width 1) (layer B.Cu) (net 17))
 (segment (start 140.8811 108.5596) (end 120.3071 108.5596) (width 1) (layer F.Cu) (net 16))
 (segment (start 110.9091 125.0696) (end 113.7031 127.8636) (width 1) (layer B.Cu) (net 16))
 (segment (start 110.1471 125.0696) (end 110.9091 125.0696) (width 1) (layer B.Cu) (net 16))
 (segment (start 107.6071 122.5296) (end 110.1471 125.0696) (width 1) (layer B.Cu) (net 16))
 (via (at 107.6071 122.5296) (size 1) (drill 0.5) (layers F.Cu B.Cu) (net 16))
 (segment (start 112.9411 122.5296) (end 107.6071 122.5296) (width 1) (layer F.Cu) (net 16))
 (segment (start 116.4971 118.9736) (end 112.9411 122.5296) (width 1) (layer F.Cu) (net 16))
 (segment (start 116.4971 112.3696) (end 116.4971 118.9736) (width 1) (layer F.Cu) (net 16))
 (segment (start 120.3071 108.5596) (end 116.4971 112.3696) (width 1) (layer F.Cu) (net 16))
 (segment (start 156.1211 116.1796) (end 155.6258 116.1796) (width 0.5) (layer F.Cu) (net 13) (status 30)))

